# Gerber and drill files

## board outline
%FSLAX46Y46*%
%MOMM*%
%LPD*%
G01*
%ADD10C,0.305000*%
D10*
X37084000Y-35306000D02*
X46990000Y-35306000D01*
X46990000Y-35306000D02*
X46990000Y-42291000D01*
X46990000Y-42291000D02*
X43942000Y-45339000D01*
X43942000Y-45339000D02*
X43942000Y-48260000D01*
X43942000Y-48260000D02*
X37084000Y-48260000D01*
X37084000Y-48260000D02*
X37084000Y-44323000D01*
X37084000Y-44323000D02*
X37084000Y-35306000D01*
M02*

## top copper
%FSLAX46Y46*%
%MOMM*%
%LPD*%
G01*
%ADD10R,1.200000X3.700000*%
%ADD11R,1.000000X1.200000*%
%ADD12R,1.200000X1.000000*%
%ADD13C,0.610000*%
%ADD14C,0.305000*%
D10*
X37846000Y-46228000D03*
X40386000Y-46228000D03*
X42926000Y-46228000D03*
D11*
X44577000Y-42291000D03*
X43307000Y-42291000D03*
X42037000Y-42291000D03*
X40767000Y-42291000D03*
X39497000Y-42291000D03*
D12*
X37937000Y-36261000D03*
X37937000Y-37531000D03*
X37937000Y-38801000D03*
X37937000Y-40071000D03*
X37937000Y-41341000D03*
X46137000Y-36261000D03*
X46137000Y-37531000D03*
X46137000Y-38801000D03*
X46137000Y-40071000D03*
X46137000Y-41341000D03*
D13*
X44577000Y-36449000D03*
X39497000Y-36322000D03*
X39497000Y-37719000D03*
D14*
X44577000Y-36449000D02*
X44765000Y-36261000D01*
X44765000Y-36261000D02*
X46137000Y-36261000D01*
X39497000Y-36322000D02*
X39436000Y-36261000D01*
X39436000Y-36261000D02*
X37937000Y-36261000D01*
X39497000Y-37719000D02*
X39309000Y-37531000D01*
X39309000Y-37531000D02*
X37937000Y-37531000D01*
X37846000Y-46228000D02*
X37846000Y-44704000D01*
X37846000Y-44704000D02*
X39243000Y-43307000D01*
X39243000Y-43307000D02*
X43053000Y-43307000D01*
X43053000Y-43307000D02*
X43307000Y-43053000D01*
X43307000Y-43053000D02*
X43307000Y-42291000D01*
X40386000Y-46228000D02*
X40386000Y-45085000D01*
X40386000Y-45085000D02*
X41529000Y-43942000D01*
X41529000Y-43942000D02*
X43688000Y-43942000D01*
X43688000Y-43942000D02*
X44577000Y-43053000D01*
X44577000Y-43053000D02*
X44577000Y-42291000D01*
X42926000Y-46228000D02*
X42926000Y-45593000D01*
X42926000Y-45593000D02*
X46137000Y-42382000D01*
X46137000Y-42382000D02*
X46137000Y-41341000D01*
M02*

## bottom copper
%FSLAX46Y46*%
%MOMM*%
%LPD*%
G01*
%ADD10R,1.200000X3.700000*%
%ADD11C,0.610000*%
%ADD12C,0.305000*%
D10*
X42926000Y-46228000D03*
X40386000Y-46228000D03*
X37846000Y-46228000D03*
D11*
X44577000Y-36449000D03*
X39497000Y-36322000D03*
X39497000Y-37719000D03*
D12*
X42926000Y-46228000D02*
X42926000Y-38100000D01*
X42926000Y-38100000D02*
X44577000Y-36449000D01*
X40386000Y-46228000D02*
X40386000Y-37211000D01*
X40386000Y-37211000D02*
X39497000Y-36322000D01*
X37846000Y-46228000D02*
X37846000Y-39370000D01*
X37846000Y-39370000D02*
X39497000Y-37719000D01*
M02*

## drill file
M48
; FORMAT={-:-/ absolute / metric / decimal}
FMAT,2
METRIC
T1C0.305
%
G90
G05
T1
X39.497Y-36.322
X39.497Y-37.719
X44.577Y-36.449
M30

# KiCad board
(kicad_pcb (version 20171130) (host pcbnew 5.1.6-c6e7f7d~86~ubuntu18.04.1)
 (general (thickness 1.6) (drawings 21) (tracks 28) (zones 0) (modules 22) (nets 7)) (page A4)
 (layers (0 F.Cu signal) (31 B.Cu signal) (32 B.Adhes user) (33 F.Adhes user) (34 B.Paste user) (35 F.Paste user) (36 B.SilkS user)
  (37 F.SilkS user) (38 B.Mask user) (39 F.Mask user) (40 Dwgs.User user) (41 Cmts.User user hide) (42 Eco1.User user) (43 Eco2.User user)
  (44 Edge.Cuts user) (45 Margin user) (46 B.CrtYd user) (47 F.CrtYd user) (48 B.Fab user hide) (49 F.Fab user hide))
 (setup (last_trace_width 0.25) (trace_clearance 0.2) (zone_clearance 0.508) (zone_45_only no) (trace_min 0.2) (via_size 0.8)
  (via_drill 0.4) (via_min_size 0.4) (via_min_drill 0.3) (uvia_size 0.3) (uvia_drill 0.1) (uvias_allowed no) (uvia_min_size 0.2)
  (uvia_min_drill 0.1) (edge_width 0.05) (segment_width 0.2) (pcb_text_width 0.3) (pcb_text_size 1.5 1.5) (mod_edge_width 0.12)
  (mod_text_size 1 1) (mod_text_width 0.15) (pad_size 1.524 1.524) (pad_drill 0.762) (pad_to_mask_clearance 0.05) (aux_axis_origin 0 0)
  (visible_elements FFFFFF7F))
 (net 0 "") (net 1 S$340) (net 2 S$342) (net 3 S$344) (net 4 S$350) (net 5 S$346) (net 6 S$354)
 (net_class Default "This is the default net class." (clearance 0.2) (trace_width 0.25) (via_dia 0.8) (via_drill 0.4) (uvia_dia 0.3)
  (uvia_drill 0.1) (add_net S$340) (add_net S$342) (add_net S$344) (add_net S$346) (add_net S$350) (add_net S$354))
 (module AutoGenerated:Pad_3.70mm (layer F.Cu) (at 37.846 46.228)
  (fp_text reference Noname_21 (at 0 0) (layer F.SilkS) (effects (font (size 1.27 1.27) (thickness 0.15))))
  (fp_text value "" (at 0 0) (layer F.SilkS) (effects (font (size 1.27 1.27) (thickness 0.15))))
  (pad 1 smd rect (at 0 0 90) (size 3.7 1.2) (layers F.Cu F.Paste F.Mask) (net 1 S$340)))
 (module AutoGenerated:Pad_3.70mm (layer F.Cu) (at 40.386 46.228)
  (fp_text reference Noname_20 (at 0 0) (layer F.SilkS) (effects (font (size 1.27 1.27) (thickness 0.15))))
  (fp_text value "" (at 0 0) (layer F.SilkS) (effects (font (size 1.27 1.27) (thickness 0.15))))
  (pad 1 smd rect (at 0 0 90) (size 3.7 1.2) (layers F.Cu F.Paste F.Mask) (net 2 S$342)))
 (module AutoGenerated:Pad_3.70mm (layer F.Cu) (at 42.926 46.228)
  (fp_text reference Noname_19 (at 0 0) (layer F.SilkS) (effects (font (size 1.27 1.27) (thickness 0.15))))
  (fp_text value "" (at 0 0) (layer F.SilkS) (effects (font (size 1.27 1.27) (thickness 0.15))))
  (pad 1 smd rect (at 0 0 90) (size 3.7 1.2) (layers F.Cu F.Paste F.Mask) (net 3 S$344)))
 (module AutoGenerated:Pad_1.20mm (layer F.Cu) (at 44.577 42.291)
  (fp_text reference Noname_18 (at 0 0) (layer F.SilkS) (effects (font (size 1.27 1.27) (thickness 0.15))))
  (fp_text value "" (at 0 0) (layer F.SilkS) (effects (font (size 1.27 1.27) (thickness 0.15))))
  (pad 15 smd rect (at 0 0 270) (size 1.2 1) (layers F.Cu F.Paste F.Mask) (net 2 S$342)))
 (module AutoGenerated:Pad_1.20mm (layer F.Cu) (at 43.307 42.291)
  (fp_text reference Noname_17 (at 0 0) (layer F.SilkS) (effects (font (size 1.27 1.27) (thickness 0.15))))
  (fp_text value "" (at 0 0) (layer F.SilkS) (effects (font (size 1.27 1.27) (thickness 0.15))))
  (pad 14 smd rect (at 0 0 270) (size 1.2 1) (layers F.Cu F.Paste F.Mask) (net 1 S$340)))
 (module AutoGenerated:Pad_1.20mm (layer F.Cu) (at 42.037 42.291)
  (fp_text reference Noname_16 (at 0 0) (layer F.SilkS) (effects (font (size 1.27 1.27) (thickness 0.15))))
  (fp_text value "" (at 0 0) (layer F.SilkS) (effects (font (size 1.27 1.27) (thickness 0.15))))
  (pad 13 smd rect (at 0 0 270) (size 1.2 1) (layers F.Cu F.Paste F.Mask)))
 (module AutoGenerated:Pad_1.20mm (layer F.Cu) (at 40.767 42.291)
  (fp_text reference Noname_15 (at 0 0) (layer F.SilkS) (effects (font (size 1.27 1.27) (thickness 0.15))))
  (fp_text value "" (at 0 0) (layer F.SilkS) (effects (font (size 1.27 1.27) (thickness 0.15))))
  (pad 12 smd rect (at 0 0 270) (size 1.2 1) (layers F.Cu F.Paste F.Mask)))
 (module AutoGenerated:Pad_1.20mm (layer F.Cu) (at 39.497 42.291)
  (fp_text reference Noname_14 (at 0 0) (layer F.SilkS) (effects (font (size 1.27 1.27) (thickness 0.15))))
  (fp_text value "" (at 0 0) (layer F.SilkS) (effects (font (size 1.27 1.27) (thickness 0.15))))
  (pad 11 smd rect (at 0 0 270) (size 1.2 1) (layers F.Cu F.Paste F.Mask)))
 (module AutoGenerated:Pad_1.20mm (layer F.Cu) (at 37.937 36.261)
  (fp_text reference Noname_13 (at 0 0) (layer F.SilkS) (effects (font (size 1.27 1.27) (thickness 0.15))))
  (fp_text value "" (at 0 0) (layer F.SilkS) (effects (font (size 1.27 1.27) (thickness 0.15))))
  (pad 1 smd rect (at 0 0) (size 1.2 1) (layers F.Cu F.Paste F.Mask) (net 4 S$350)))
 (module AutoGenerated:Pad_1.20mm (layer F.Cu) (at 37.937 37.531)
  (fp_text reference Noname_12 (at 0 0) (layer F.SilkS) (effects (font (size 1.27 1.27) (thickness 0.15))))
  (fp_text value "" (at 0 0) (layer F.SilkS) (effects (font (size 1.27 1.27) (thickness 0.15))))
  (pad 2 smd rect (at 0 0) (size 1.2 1) (layers F.Cu F.Paste F.Mask) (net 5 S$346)))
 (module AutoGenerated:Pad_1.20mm (layer F.Cu) (at 37.937 38.801)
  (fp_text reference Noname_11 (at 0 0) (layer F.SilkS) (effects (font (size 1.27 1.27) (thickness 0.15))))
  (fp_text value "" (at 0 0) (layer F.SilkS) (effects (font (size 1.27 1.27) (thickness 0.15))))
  (pad 3 smd rect (at 0 0) (size 1.2 1) (layers F.Cu F.Paste F.Mask)))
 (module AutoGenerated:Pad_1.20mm (layer F.Cu) (at 37.937 40.071)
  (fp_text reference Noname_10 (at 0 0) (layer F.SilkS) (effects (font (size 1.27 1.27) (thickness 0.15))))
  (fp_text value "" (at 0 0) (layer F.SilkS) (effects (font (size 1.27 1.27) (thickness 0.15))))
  (pad 4 smd rect (at 0 0) (size 1.2 1) (layers F.Cu F.Paste F.Mask)))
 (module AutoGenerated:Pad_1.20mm (layer F.Cu) (at 37.937 41.341)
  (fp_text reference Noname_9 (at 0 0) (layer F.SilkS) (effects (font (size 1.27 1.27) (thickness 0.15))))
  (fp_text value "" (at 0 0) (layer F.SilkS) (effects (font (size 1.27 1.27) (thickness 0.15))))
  (pad 5 smd rect (at 0 0) (size 1.2 1) (layers F.Cu F.Paste F.Mask)))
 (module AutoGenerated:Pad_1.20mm (layer F.Cu) (at 46.137 36.261)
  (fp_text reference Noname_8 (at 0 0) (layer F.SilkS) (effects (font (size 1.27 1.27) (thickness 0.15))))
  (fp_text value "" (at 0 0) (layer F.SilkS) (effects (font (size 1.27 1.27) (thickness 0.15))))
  (pad 6 smd rect (at 0 0) (size 1.2 1) (layers F.Cu F.Paste F.Mask) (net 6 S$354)))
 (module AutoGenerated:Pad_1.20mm (layer F.Cu) (at 46.137 37.531)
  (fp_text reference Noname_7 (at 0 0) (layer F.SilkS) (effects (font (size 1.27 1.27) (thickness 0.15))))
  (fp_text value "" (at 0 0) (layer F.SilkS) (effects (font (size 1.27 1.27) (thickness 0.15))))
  (pad 7 smd rect (at 0 0) (size 1.2 1) (layers F.Cu F.Paste F.Mask)))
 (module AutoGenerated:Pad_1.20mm (layer F.Cu) (at 46.137 38.801)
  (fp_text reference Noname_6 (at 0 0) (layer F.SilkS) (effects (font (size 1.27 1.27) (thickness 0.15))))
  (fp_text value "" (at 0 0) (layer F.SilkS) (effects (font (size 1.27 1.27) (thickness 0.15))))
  (pad 8 smd rect (at 0 0) (size 1.2 1) (layers F.Cu F.Paste F.Mask)))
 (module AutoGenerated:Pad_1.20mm (layer F.Cu) (at 46.137 40.071)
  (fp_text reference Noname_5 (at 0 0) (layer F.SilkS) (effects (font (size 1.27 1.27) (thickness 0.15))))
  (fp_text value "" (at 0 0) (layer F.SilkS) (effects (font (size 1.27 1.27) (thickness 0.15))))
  (pad 9 smd rect (at 0 0) (size 1.2 1) (layers F.Cu F.Paste F.Mask)))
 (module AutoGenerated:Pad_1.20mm (layer F.Cu) (at 46.137 41.341)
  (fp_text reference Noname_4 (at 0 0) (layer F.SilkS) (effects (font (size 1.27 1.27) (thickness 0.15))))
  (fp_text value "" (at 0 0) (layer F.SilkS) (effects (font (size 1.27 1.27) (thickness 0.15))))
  (pad 10 smd rect (at 0 0) (size 1.2 1) (layers F.Cu F.Paste F.Mask) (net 3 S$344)))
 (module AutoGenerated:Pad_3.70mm (layer F.Cu) (at 42.926 46.228)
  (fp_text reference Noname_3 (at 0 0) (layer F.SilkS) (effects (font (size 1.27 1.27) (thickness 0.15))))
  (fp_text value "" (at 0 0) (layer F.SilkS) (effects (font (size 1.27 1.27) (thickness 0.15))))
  (pad 1 smd rect (at 0 0 90) (size 3.7 1.2) (layers B.Cu B.Paste B.Mask) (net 6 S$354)))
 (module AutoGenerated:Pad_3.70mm (layer F.Cu) (at 40.386 46.228)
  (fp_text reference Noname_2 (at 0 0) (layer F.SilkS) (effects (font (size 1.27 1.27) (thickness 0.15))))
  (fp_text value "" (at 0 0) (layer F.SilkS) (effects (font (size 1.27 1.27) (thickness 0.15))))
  (pad 1 smd rect (at 0 0 90) (size 3.7 1.2) (layers B.Cu B.Paste B.Mask) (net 4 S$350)))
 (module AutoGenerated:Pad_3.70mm (layer F.Cu) (at 37.846 46.228)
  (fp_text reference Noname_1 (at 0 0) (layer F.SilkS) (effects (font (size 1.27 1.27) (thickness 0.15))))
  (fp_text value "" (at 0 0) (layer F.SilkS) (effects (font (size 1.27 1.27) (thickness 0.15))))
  (pad 1 smd rect (at 0 0 90) (size 3.7 1.2) (layers B.Cu B.Paste B.Mask) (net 5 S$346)))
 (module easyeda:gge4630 (layer F.Cu) (at 42.037 37.719)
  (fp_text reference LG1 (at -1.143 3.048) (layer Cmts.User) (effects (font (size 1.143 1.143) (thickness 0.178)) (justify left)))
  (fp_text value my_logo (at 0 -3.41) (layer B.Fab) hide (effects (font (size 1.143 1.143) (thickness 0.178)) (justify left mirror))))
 (gr_line (start 37.084 35.306) (end 46.99 35.306) (layer Edge.Cuts) (width 0.305))
 (gr_line (start 46.99 35.306) (end 46.99 42.291) (layer Edge.Cuts) (width 0.305))
 (gr_line (start 46.99 42.291) (end 43.942 45.339) (layer Edge.Cuts) (width 0.305))
 (gr_line (start 43.942 45.339) (end 43.942 48.26) (layer Edge.Cuts) (width 0.305))
 (gr_line (start 43.942 48.26) (end 37.084 48.26) (layer Edge.Cuts) (width 0.305))
 (gr_line (start 37.084 48.26) (end 37.084 44.323) (layer Edge.Cuts) (width 0.305))
 (gr_line (start 37.084 44.323) (end 37.084 35.306) (layer Edge.Cuts) (width 0.305))
 (segment (start 42.926 46.228) (end 42.926 38.1) (width 0.305) (layer B.Cu) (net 6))
 (segment (start 42.926 38.1) (end 44.577 36.449) (width 0.305) (layer B.Cu) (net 6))
 (segment (start 44.577 36.449) (end 44.765 36.261) (width 0.305) (layer F.Cu) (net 6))
 (segment (start 44.765 36.261) (end 46.137 36.261) (width 0.305) (layer F.Cu) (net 6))
 (segment (start 40.386 46.228) (end 40.386 37.211) (width 0.305) (layer B.Cu) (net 4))
 (segment (start 40.386 37.211) (end 39.497 36.322) (width 0.305) (layer B.Cu) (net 4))
 (segment (start 39.497 36.322) (end 39.436 36.261) (width 0.305) (layer F.Cu) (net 4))
 (segment (start 39.436 36.261) (end 37.937 36.261) (width 0.305) (layer F.Cu) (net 4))
 (segment (start 37.846 46.228) (end 37.846 39.37) (width 0.305) (layer B.Cu) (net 5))
 (segment (start 37.846 39.37) (end 39.497 37.719) (width 0.305) (layer B.Cu) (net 5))
 (segment (start 39.497 37.719) (end 39.309 37.531) (width 0.305) (layer F.Cu) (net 5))
 (segment (start 39.309 37.531) (end 37.937 37.531) (width 0.305) (layer F.Cu) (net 5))
 (segment (start 37.846 46.228) (end 37.846 44.704) (width 0.305) (layer F.Cu) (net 1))
 (segment (start 37.846 44.704) (end 39.243 43.307) (width 0.305) (layer F.Cu) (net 1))
 (segment (start 39.243 43.307) (end 43.053 43.307) (width 0.305) (layer F.Cu) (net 1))
 (segment (start 43.053 43.307) (end 43.307 43.053) (width 0.305) (layer F.Cu) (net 1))
 (segment (start 43.307 43.053) (end 43.307 42.291) (width 0.305) (layer F.Cu) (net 1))
 (segment (start 40.386 46.228) (end 40.386 45.085) (width 0.305) (layer F.Cu) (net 2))
 (segment (start 40.386 45.085) (end 41.529 43.942) (width 0.305) (layer F.Cu) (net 2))
 (segment (start 41.529 43.942) (end 43.688 43.942) (width 0.305) (layer F.Cu) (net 2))
 (segment (start 43.688 43.942) (end 44.577 43.053) (width 0.305) (layer F.Cu) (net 2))
 (segment (start 44.577 43.053) (end 44.577 42.291) (width 0.305) (layer F.Cu) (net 2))
 (segment (start 42.926 46.228) (end 42.926 45.593) (width 0.305) (layer F.Cu) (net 3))
 (segment (start 42.926 45.593) (end 46.137 42.382) (width 0.305) (layer F.Cu) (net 3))
 (segment (start 46.137 42.382) (end 46.137 41.341) (width 0.305) (layer F.Cu) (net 3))
 (via (at 44.577 36.449) (size 0.61) (drill 0.305) (layers F.Cu B.Cu) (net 6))
 (via (at 39.497 36.322) (size 0.61) (drill 0.305) (layers F.Cu B.Cu) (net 4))
 (via (at 39.497 37.719) (size 0.61) (drill 0.305) (layers F.Cu B.Cu) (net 5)))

